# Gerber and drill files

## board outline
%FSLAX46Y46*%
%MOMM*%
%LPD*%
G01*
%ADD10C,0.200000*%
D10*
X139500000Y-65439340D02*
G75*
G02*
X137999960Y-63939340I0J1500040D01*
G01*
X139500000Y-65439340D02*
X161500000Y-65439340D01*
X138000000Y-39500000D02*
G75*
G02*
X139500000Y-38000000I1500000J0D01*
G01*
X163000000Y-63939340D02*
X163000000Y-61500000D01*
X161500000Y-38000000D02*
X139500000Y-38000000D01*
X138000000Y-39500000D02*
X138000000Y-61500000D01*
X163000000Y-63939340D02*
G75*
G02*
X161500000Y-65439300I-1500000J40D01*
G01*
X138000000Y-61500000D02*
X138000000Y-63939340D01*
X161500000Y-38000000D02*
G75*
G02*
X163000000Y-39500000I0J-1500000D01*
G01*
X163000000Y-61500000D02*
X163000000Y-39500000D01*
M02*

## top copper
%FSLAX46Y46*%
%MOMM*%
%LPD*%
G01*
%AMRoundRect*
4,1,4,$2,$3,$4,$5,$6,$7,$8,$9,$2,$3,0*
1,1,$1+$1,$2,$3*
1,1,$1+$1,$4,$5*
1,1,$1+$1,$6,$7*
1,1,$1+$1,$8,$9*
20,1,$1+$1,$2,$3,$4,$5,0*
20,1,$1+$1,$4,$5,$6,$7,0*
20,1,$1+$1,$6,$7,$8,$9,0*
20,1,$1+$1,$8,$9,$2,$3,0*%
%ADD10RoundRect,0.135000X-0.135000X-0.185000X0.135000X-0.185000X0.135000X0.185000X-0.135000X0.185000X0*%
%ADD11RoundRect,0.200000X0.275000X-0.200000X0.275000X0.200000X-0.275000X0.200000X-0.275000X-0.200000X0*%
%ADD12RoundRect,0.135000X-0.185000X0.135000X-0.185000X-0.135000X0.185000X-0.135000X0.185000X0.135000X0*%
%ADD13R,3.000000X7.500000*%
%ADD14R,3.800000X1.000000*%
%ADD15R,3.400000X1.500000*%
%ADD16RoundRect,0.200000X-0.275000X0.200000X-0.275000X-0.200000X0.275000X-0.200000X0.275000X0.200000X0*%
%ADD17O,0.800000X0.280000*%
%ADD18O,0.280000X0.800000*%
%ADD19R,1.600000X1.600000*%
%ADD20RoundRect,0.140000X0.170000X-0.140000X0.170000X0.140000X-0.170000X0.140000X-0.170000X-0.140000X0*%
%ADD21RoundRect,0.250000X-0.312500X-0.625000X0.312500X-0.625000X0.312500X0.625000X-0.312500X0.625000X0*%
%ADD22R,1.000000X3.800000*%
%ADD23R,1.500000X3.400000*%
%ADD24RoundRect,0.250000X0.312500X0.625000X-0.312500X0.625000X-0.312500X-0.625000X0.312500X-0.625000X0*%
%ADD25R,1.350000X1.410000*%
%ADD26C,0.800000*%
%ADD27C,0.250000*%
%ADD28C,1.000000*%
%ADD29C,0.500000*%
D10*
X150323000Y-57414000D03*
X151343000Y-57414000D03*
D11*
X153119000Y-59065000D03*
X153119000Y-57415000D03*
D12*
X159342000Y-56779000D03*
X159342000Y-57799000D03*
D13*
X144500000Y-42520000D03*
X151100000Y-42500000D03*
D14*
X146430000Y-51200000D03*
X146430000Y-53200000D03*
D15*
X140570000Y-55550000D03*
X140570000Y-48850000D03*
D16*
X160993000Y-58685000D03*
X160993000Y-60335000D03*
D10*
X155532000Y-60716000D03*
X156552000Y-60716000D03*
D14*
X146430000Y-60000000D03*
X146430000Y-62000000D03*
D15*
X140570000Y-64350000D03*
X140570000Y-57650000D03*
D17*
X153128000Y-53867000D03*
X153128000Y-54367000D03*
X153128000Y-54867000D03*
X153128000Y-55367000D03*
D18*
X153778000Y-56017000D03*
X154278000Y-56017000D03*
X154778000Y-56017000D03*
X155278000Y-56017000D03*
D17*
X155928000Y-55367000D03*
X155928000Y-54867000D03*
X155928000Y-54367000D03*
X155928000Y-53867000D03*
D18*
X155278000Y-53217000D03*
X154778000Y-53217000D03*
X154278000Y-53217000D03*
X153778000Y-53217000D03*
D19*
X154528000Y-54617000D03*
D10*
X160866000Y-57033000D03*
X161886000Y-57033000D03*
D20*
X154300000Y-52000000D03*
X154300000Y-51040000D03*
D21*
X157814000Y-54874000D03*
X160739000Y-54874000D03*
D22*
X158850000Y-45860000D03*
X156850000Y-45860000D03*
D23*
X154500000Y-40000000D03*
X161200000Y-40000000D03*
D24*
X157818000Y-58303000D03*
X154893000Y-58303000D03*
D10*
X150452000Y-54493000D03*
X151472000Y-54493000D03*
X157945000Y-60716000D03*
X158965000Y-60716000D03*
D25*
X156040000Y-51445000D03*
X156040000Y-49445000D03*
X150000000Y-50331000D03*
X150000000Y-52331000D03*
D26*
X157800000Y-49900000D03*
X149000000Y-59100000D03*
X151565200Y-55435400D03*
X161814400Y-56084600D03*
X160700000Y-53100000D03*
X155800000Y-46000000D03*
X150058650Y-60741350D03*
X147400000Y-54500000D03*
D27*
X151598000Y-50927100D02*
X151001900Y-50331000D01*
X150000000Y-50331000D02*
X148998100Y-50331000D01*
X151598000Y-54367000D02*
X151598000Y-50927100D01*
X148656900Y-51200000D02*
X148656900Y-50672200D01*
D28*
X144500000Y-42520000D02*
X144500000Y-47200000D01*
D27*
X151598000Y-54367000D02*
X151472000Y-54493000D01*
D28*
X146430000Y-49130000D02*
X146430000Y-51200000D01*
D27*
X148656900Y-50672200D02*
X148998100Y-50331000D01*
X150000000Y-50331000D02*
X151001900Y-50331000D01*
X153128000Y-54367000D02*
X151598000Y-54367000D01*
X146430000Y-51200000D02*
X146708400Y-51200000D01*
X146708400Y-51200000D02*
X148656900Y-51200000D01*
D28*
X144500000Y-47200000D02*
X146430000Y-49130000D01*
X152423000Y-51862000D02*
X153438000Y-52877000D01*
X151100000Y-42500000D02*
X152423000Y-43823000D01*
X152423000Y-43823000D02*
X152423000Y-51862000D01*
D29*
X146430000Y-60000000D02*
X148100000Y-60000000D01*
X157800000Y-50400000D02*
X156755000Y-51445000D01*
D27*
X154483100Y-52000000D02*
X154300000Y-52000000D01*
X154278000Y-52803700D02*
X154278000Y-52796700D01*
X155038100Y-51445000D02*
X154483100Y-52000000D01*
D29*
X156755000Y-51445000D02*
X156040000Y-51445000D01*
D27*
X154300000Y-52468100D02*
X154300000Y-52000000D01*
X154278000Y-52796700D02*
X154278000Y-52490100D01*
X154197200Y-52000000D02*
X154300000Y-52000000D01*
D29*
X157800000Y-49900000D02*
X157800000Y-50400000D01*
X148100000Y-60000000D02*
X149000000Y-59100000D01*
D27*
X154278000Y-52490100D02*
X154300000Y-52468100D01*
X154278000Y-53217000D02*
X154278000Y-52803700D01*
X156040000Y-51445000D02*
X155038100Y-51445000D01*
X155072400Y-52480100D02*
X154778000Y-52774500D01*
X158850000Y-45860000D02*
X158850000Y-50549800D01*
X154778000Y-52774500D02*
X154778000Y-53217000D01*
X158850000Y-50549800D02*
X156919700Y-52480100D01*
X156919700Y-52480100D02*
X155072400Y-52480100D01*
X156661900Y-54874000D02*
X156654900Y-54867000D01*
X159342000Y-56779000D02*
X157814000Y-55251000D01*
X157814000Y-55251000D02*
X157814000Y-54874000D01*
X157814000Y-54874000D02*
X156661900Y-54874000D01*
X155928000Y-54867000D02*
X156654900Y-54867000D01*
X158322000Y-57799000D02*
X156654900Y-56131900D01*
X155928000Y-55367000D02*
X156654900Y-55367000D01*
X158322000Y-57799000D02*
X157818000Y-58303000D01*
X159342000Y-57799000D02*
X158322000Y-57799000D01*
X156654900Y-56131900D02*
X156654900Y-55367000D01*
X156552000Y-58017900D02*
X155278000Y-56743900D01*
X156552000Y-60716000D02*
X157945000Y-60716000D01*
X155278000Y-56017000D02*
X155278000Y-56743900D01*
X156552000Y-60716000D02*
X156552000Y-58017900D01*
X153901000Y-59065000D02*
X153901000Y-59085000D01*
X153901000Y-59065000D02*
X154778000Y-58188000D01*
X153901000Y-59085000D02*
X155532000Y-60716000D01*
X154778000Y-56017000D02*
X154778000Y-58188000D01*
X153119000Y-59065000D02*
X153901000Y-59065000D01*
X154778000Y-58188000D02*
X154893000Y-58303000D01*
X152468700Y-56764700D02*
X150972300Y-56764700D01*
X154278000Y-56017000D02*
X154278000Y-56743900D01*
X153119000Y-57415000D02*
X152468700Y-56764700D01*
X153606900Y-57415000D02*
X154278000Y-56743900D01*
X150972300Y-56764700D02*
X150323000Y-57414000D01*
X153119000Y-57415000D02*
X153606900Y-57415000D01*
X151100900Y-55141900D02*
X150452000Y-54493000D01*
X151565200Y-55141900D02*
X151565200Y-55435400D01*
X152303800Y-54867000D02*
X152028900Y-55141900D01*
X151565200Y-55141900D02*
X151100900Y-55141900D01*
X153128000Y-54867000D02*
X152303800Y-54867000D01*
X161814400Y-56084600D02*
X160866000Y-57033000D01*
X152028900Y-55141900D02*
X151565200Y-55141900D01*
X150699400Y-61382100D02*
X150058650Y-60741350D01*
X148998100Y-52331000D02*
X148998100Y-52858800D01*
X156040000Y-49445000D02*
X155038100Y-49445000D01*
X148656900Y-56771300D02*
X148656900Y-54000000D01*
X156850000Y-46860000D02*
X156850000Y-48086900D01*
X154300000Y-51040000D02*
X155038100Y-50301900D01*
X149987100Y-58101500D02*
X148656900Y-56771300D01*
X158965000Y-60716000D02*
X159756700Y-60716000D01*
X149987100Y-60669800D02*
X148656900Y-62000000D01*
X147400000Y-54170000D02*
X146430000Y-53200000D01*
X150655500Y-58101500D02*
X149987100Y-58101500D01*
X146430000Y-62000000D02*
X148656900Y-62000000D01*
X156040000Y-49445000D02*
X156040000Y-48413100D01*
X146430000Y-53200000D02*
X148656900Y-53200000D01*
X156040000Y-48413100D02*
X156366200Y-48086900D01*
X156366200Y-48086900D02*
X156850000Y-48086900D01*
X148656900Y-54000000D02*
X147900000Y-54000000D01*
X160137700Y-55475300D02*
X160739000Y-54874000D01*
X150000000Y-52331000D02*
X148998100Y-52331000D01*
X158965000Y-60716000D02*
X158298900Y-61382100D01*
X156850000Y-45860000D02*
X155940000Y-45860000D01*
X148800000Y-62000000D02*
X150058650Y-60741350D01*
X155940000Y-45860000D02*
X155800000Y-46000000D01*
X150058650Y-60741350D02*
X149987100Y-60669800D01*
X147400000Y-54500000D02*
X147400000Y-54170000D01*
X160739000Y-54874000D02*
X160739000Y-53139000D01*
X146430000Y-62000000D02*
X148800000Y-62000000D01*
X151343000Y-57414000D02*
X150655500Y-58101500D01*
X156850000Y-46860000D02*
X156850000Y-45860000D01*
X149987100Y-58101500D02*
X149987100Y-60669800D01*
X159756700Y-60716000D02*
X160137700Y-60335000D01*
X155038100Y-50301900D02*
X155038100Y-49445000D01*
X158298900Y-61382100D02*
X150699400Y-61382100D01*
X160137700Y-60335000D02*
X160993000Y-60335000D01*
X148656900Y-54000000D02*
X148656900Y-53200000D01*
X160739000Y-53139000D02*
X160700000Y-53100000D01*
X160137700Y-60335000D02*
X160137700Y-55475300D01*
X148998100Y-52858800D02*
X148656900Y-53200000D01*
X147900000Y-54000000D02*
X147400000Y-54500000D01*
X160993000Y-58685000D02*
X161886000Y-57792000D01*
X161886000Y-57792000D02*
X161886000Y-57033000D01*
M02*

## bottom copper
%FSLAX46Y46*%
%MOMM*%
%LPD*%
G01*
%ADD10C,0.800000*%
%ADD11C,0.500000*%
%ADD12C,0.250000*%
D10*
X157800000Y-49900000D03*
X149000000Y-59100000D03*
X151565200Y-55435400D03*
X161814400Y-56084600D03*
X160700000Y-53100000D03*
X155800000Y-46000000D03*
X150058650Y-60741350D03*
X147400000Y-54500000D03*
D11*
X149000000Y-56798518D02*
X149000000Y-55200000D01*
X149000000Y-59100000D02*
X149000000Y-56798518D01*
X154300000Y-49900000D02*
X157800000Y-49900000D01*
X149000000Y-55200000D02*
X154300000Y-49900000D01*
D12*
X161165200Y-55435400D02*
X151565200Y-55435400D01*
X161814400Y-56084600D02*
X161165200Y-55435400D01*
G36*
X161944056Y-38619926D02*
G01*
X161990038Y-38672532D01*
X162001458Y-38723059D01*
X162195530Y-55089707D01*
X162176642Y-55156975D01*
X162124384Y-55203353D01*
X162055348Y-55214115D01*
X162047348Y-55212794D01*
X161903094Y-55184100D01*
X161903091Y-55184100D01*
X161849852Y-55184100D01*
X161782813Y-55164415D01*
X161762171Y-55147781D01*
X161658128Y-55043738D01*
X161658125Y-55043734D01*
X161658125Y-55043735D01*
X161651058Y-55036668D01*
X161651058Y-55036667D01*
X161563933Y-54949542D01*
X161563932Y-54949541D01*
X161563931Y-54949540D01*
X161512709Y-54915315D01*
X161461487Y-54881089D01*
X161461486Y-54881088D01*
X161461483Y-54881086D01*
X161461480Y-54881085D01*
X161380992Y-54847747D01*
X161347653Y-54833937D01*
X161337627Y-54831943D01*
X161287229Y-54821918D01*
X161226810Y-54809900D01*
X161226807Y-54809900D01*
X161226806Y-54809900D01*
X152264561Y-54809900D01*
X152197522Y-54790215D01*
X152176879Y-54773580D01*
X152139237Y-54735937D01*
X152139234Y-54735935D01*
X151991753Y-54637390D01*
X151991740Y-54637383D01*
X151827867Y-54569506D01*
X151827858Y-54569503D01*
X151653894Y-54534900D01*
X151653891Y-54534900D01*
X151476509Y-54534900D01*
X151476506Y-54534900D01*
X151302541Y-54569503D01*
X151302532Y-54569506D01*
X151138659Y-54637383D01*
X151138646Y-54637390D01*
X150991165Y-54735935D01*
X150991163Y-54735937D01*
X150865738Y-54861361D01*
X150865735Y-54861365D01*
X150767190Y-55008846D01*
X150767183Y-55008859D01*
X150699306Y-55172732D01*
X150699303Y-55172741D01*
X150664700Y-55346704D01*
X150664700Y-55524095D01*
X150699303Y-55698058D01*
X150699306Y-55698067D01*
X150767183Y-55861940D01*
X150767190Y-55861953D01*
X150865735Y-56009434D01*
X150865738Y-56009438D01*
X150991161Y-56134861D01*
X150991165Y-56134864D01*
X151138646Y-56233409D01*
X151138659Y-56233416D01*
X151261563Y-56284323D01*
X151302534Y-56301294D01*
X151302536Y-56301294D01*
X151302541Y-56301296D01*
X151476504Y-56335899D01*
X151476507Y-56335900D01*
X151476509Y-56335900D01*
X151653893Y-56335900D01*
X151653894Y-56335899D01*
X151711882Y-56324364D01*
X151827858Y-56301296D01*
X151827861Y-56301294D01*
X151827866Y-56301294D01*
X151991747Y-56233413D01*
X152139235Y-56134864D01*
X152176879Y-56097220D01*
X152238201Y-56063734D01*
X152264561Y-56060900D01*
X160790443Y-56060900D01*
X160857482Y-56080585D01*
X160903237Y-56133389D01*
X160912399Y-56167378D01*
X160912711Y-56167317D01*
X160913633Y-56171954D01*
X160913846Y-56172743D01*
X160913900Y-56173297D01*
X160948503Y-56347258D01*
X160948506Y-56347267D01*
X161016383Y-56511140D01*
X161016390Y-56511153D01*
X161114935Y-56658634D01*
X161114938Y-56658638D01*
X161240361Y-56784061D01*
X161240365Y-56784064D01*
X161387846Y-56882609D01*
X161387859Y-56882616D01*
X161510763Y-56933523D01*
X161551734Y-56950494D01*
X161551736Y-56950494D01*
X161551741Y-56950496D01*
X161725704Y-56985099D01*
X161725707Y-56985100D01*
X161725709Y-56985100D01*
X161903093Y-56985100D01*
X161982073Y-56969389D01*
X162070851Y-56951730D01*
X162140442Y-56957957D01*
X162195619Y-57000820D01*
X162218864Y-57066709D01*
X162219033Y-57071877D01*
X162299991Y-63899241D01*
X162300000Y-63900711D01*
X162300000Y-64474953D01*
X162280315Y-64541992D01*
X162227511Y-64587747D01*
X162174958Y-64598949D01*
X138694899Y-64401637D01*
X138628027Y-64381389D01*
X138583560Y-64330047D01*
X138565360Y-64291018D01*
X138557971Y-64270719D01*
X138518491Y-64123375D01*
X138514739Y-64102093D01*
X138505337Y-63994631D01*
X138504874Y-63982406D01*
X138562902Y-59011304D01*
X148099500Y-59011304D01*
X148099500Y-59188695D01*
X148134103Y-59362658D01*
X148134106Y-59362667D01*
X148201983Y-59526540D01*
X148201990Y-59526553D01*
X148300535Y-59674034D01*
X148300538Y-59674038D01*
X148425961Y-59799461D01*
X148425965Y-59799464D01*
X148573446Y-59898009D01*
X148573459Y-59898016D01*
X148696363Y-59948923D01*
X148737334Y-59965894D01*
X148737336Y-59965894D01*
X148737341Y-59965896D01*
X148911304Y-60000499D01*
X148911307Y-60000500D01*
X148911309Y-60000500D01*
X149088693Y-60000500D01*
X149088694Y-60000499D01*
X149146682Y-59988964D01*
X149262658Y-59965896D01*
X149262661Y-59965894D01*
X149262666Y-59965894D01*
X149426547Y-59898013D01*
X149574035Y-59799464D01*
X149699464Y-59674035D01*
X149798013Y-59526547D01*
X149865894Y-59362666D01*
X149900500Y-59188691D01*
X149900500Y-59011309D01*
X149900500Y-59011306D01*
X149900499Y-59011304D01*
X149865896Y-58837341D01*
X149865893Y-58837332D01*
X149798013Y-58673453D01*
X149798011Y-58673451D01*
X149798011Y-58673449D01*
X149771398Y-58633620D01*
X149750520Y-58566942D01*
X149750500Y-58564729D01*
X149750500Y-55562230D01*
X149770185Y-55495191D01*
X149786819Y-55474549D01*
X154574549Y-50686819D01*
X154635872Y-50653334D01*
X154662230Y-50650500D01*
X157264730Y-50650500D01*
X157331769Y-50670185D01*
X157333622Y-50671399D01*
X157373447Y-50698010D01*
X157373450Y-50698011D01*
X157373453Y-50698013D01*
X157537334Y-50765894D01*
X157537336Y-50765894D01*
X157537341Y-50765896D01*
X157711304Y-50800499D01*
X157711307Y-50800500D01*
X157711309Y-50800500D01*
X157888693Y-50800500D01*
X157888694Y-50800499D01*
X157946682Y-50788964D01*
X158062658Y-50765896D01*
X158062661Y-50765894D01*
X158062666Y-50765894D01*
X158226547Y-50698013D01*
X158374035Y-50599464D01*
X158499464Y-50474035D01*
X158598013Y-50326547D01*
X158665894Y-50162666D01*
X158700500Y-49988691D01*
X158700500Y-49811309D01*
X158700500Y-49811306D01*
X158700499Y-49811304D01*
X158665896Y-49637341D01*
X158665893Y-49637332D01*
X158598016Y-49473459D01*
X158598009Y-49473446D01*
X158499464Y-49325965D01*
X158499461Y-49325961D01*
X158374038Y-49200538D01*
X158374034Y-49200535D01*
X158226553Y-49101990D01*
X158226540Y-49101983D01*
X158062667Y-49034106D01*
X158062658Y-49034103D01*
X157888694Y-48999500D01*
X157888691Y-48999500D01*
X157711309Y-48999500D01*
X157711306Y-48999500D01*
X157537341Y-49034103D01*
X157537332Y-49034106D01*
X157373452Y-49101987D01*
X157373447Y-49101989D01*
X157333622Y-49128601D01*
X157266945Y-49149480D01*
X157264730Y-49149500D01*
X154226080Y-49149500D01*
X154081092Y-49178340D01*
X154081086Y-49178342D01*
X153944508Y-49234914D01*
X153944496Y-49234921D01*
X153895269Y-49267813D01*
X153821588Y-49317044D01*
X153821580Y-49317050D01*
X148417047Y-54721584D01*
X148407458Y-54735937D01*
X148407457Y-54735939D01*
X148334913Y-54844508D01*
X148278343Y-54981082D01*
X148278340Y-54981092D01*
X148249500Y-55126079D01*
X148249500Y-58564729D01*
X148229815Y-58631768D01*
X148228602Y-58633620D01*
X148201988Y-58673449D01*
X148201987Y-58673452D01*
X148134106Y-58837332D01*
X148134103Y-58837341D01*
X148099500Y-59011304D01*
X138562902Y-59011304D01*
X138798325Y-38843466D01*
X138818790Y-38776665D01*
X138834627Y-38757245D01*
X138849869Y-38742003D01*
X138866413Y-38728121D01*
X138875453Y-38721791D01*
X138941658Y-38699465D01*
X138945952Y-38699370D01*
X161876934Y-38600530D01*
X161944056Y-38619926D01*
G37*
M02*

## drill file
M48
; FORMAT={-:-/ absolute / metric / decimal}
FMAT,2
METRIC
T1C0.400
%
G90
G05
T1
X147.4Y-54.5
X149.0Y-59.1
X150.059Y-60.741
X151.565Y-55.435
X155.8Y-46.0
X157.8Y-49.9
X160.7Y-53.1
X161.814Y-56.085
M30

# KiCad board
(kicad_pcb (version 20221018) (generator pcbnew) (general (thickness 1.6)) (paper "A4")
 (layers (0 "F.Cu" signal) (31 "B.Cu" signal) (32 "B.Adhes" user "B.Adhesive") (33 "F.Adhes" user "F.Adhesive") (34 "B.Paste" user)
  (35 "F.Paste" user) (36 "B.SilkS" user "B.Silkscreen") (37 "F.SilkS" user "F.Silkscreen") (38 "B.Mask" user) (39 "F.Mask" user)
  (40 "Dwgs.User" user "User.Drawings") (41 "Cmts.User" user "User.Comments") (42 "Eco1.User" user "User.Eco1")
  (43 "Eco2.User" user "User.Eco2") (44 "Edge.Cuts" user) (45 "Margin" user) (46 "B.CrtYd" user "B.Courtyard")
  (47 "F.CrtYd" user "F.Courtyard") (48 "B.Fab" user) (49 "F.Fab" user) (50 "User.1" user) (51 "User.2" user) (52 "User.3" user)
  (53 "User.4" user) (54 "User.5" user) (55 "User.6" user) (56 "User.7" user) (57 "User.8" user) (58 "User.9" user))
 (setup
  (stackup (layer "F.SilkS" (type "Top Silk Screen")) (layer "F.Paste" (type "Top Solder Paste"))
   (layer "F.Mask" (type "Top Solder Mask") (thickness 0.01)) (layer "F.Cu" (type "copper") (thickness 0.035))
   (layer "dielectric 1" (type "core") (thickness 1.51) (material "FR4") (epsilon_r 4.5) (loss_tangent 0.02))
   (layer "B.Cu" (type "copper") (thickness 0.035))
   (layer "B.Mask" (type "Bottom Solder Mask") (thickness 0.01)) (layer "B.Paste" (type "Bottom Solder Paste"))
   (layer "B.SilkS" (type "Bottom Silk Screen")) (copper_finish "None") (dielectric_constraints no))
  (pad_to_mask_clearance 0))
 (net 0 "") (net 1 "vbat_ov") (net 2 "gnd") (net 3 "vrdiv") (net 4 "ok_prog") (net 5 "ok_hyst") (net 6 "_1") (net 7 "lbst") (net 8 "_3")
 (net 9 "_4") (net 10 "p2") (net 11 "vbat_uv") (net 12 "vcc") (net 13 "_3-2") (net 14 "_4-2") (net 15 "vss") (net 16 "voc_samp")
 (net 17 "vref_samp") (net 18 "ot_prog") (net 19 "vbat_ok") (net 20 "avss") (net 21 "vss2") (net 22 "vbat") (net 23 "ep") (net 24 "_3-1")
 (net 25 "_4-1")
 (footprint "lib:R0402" (layer "F.Cu") (at 150.833 57.414)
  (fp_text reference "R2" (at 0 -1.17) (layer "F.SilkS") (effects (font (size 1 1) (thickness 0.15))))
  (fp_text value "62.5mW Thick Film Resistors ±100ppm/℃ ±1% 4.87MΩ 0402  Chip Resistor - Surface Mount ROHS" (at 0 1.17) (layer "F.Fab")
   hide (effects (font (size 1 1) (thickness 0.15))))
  (pad "1" smd roundrect (at -0.51 0) (size 0.54 0.64) (layers "F.Cu" "F.Paste" "F.Mask") (roundrect_rratio 0.25) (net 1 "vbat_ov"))
  (pad "2" smd roundrect (at 0.51 0) (size 0.54 0.64) (layers "F.Cu" "F.Paste" "F.Mask") (roundrect_rratio 0.25) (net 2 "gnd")))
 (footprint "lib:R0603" (layer "F.Cu") (at 153.119 58.24 90)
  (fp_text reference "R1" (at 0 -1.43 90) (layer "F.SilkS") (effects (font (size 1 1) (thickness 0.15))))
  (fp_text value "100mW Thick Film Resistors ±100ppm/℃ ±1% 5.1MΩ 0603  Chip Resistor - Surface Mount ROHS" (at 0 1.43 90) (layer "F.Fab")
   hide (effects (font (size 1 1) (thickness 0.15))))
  (pad "1" smd roundrect (at -0.825 0 90) (size 0.8 0.95) (layers "F.Cu" "F.Paste" "F.Mask") (roundrect_rratio 0.25) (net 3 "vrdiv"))
  (pad "2" smd roundrect (at 0.825 0 90) (size 0.8 0.95) (layers "F.Cu" "F.Paste" "F.Mask") (roundrect_rratio 0.25) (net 1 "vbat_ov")))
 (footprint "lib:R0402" (layer "F.Cu") (at 159.342 57.289 -90)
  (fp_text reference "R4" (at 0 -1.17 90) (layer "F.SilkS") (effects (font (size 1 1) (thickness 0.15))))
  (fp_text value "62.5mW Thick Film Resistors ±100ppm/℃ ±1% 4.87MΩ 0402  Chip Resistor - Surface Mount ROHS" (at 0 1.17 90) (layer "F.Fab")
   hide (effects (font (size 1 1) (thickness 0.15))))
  (pad "1" smd roundrect (at -0.51 0 270) (size 0.54 0.64) (layers "F.Cu" "F.Paste" "F.Mask") (roundrect_rratio 0.25) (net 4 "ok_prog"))
  (pad "2" smd roundrect (at 0.51 0 270) (size 0.54 0.64) (layers "F.Cu" "F.Paste" "F.Mask") (roundrect_rratio 0.25) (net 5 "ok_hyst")))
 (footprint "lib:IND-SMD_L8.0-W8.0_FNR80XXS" (layer "F.Cu") (at 147.8 42.51)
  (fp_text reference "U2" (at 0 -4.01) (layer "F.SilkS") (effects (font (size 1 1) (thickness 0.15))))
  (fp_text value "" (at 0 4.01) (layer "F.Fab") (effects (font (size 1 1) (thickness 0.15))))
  (pad "1" smd rect (at -3.3 0.01) (size 3 7.5) (layers "F.Cu" "F.Paste" "F.Mask") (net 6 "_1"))
  (pad "2" smd rect (at 3.3 -0.01) (size 3 7.5) (layers "F.Cu" "F.Paste" "F.Mask") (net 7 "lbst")))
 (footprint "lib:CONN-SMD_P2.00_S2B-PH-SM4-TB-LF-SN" (layer "F.Cu") (at 143.5 52.2 -90)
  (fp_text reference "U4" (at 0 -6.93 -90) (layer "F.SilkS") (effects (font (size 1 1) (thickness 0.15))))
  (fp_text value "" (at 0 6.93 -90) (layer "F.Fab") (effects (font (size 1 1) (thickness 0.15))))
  (pad "1" smd rect (at -1 -2.93 270) (size 1 3.8) (layers "F.Cu" "F.Paste" "F.Mask") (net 6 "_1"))
  (pad "2" smd rect (at 1 -2.93 270) (size 1 3.8) (layers "F.Cu" "F.Paste" "F.Mask") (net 2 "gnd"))
  (pad "3" smd rect (at 3.35 2.93 270) (size 1.5 3.4) (layers "F.Cu" "F.Paste" "F.Mask") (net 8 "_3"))
  (pad "4" smd rect (at -3.35 2.93 270) (size 1.5 3.4) (layers "F.Cu" "F.Paste" "F.Mask") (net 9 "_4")))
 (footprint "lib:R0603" (layer "F.Cu") (at 160.993 59.51 -90)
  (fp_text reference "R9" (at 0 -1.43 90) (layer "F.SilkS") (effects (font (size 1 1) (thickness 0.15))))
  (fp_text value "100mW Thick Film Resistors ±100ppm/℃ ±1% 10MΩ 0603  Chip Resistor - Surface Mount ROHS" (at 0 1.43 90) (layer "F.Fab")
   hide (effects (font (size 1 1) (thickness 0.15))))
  (pad "1" smd roundrect (at -0.825 0 270) (size 0.8 0.95) (layers "F.Cu" "F.Paste" "F.Mask") (roundrect_rratio 0.25) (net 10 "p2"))
  (pad "2" smd roundrect (at 0.825 0 270) (size 0.8 0.95) (layers "F.Cu" "F.Paste" "F.Mask") (roundrect_rratio 0.25) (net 2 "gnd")))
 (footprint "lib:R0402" (layer "F.Cu") (at 156.042 60.716)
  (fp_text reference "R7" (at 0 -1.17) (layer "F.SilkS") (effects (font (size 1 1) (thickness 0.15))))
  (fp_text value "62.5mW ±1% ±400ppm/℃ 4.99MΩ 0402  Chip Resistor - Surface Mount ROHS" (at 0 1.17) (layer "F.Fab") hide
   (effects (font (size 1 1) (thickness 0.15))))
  (pad "1" smd roundrect (at -0.51 0) (size 0.54 0.64) (layers "F.Cu" "F.Paste" "F.Mask") (roundrect_rratio 0.25) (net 3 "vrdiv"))
  (pad "2" smd roundrect (at 0.51 0) (size 0.54 0.64) (layers "F.Cu" "F.Paste" "F.Mask") (roundrect_rratio 0.25) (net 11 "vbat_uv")))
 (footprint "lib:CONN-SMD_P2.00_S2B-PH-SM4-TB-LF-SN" (layer "F.Cu") (at 143.5 61 -90)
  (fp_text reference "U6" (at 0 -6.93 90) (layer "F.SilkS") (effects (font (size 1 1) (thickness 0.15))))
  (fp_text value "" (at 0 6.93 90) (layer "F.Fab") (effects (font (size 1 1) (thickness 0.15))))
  (pad "1" smd rect (at -1 -2.93 270) (size 1 3.8) (layers "F.Cu" "F.Paste" "F.Mask") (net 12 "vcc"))
  (pad "2" smd rect (at 1 -2.93 270) (size 1 3.8) (layers "F.Cu" "F.Paste" "F.Mask") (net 2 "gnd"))
  (pad "3" smd rect (at 3.35 2.93 270) (size 1.5 3.4) (layers "F.Cu" "F.Paste" "F.Mask") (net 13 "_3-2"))
  (pad "4" smd rect (at -3.35 2.93 270) (size 1.5 3.4) (layers "F.Cu" "F.Paste" "F.Mask") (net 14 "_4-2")))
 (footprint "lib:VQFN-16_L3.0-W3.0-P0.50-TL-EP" (layer "F.Cu") (at 154.528 54.617)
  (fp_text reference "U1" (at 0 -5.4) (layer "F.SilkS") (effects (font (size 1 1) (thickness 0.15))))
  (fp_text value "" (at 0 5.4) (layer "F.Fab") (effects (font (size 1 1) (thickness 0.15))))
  (pad "1" smd oval (at -1.4 -0.75 90) (size 0.28 0.8) (layers "F.Cu" "F.Paste" "F.Mask") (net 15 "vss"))
  (pad "2" smd oval (at -1.4 -0.25 90) (size 0.28 0.8) (layers "F.Cu" "F.Paste" "F.Mask") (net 6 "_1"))
  (pad "3" smd oval (at -1.4 0.25 90) (size 0.28 0.8) (layers "F.Cu" "F.Paste" "F.Mask") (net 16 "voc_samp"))
  (pad "4" smd oval (at -1.4 0.75 90) (size 0.28 0.8) (layers "F.Cu" "F.Paste" "F.Mask") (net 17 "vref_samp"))
  (pad "5" smd oval (at -0.75 1.4) (size 0.28 0.8) (layers "F.Cu" "F.Paste" "F.Mask") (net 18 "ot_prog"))
  (pad "6" smd oval (at -0.25 1.4) (size 0.28 0.8) (layers "F.Cu" "F.Paste" "F.Mask") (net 1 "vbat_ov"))
  (pad "7" smd oval (at 0.25 1.4) (size 0.28 0.8) (layers "F.Cu" "F.Paste" "F.Mask") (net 3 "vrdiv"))
  (pad "8" smd oval (at 0.75 1.4) (size 0.28 0.8) (layers "F.Cu" "F.Paste" "F.Mask") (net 11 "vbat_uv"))
  (pad "9" smd oval (at 1.4 0.75 90) (size 0.28 0.8) (layers "F.Cu" "F.Paste" "F.Mask") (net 5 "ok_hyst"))
  (pad "10" smd oval (at 1.4 0.25 90) (size 0.28 0.8) (layers "F.Cu" "F.Paste" "F.Mask") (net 4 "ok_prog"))
  (pad "11" smd oval (at 1.4 -0.25 90) (size 0.28 0.8) (layers "F.Cu" "F.Paste" "F.Mask") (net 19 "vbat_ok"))
  (pad "12" smd oval (at 1.4 -0.75 90) (size 0.28 0.8) (layers "F.Cu" "F.Paste" "F.Mask") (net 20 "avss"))
  (pad "13" smd oval (at 0.75 -1.4) (size 0.28 0.8) (layers "F.Cu" "F.Paste" "F.Mask") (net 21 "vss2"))
  (pad "14" smd oval (at 0.25 -1.4) (size 0.28 0.8) (layers "F.Cu" "F.Paste" "F.Mask") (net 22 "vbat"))
  (pad "15" smd oval (at -0.25 -1.4) (size 0.28 0.8) (layers "F.Cu" "F.Paste" "F.Mask") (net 12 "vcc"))
  (pad "16" smd oval (at -0.75 -1.4) (size 0.28 0.8) (layers "F.Cu" "F.Paste" "F.Mask") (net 7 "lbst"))
  (pad "17" smd rect (at 0 0) (size 1.6 1.6) (layers "F.Cu" "F.Paste" "F.Mask") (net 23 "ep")))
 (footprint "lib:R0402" (layer "F.Cu") (at 161.376 57.033)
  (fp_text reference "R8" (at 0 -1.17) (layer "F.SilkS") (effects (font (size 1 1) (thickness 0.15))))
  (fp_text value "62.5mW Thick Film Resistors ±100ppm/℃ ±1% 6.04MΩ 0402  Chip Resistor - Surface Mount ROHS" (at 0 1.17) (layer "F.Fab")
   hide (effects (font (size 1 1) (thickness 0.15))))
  (pad "1" smd roundrect (at -0.51 0) (size 0.54 0.64) (layers "F.Cu" "F.Paste" "F.Mask") (roundrect_rratio 0.25) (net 16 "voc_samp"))
  (pad "2" smd roundrect (at 0.51 0) (size 0.54 0.64) (layers "F.Cu" "F.Paste" "F.Mask") (roundrect_rratio 0.25) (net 10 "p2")))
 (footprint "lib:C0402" (layer "F.Cu") (at 154.3 51.52 90)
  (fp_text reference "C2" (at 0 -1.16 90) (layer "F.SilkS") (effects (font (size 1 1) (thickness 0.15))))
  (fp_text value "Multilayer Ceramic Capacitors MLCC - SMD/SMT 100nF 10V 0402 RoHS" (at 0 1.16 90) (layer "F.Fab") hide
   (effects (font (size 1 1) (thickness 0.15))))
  (pad "1" smd roundrect (at -0.48 0 90) (size 0.56 0.62) (layers "F.Cu" "F.Paste" "F.Mask") (roundrect_rratio 0.25) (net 12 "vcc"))
  (pad "2" smd roundrect (at 0.48 0 90) (size 0.56 0.62) (layers "F.Cu" "F.Paste" "F.Mask") (roundrect_rratio 0.25) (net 2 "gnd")))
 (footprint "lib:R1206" (layer "F.Cu") (at 159.2765 54.874)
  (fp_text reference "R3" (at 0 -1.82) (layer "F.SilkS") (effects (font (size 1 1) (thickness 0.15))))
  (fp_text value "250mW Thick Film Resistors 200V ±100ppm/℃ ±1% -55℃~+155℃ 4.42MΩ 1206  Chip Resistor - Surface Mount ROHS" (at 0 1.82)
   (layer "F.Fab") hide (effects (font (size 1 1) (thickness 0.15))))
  (pad "1" smd roundrect (at -1.4625 0) (size 1.125 1.75) (layers "F.Cu" "F.Paste" "F.Mask") (roundrect_rratio 0.2222222222)
   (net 4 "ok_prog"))
  (pad "2" smd roundrect (at 1.4625 0) (size 1.125 1.75) (layers "F.Cu" "F.Paste" "F.Mask") (roundrect_rratio 0.2222222222) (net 2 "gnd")))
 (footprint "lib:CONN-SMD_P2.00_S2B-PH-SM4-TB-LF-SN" (layer "F.Cu") (at 157.85 42.93 180)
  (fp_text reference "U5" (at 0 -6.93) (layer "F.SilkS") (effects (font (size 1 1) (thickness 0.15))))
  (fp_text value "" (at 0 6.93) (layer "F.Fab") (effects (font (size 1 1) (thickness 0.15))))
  (pad "1" smd rect (at -1 -2.93 180) (size 1 3.8) (layers "F.Cu" "F.Paste" "F.Mask") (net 22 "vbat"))
  (pad "2" smd rect (at 1 -2.93 180) (size 1 3.8) (layers "F.Cu" "F.Paste" "F.Mask") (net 2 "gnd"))
  (pad "3" smd rect (at 3.35 2.93 180) (size 1.5 3.4) (layers "F.Cu" "F.Paste" "F.Mask") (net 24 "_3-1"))
  (pad "4" smd rect (at -3.35 2.93 180) (size 1.5 3.4) (layers "F.Cu" "F.Paste" "F.Mask") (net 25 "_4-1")))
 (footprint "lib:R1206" (layer "F.Cu") (at 156.3555 58.303 180)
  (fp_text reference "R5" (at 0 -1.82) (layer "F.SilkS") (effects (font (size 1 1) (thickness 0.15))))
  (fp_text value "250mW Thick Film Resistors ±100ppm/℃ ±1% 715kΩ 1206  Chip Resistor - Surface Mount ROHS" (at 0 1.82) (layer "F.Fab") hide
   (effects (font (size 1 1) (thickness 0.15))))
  (pad "1" smd roundrect (at -1.4625 0 180) (size 1.125 1.75) (layers "F.Cu" "F.Paste" "F.Mask") (roundrect_rratio 0.2222222222)
   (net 5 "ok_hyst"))
  (pad "2" smd roundrect (at 1.4625 0 180) (size 1.125 1.75) (layers "F.Cu" "F.Paste" "F.Mask") (roundrect_rratio 0.2222222222)
   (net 3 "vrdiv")))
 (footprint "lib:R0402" (layer "F.Cu") (at 150.962 54.493)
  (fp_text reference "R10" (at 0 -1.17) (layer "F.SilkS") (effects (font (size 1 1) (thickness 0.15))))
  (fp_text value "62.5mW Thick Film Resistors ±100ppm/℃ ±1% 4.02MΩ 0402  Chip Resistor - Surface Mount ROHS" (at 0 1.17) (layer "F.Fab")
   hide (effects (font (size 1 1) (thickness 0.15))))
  (pad "1" smd roundrect (at -0.51 0) (size 0.54 0.64) (layers "F.Cu" "F.Paste" "F.Mask") (roundrect_rratio 0.25) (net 16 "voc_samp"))
  (pad "2" smd roundrect (at 0.51 0) (size 0.54 0.64) (layers "F.Cu" "F.Paste" "F.Mask") (roundrect_rratio 0.25) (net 6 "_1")))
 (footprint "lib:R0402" (layer "F.Cu") (at 158.455 60.716)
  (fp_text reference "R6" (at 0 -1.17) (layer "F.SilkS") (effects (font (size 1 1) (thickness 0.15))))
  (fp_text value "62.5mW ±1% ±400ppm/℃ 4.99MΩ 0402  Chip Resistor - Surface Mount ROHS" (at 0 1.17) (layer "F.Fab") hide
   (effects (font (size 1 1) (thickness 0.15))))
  (pad "1" smd roundrect (at -0.51 0) (size 0.54 0.64) (layers "F.Cu" "F.Paste" "F.Mask") (roundrect_rratio 0.25) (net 11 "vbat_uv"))
  (pad "2" smd roundrect (at 0.51 0) (size 0.54 0.64) (layers "F.Cu" "F.Paste" "F.Mask") (roundrect_rratio 0.25) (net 2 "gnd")))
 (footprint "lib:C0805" (layer "F.Cu") (at 156.04 50.445 90)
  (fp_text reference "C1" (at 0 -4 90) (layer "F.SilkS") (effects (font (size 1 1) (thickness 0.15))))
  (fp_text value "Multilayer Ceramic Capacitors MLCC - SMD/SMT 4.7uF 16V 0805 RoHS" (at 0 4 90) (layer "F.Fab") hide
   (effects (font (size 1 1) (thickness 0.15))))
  (pad "1" smd rect (at -1 0 90) (size 1.41 1.35) (layers "F.Cu" "F.Paste" "F.Mask") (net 12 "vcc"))
  (pad "2" smd rect (at 1 0 90) (size 1.41 1.35) (layers "F.Cu" "F.Paste" "F.Mask") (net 2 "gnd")))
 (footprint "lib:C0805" (layer "F.Cu") (at 150 51.331 -90)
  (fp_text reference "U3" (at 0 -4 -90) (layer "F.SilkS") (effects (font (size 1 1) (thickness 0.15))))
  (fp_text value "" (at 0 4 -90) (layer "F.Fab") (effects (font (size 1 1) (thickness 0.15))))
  (pad "1" smd rect (at -1 0 270) (size 1.41 1.35) (layers "F.Cu" "F.Paste" "F.Mask") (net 6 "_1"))
  (pad "2" smd rect (at 1 0 270) (size 1.41 1.35) (layers "F.Cu" "F.Paste" "F.Mask") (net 2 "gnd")))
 (gr_arc (start 139.5 65.43934) (mid 138.43934 65) (end 138 63.93934) (stroke (width 0.2) (type default)) (layer "Edge.Cuts"))
 (gr_line (start 139.5 65.43934) (end 161.5 65.43934) (stroke (width 0.2) (type default)) (layer "Edge.Cuts"))
 (gr_arc (start 138 39.5) (mid 138.43934 38.43934) (end 139.5 38) (stroke (width 0.2) (type default)) (layer "Edge.Cuts"))
 (gr_line (start 163 63.93934) (end 163 61.5) (stroke (width 0.2) (type default)) (layer "Edge.Cuts"))
 (gr_line (start 161.5 38) (end 139.5 38) (stroke (width 0.2) (type default)) (layer "Edge.Cuts"))
 (gr_line (start 138 39.5) (end 138 61.5) (stroke (width 0.2) (type default)) (layer "Edge.Cuts"))
 (gr_arc (start 163 63.93934) (mid 162.56066 65) (end 161.5 65.43934) (stroke (width 0.2) (type default)) (layer "Edge.Cuts"))
 (gr_line (start 138 61.5) (end 138 63.93934) (stroke (width 0.2) (type default)) (layer "Edge.Cuts"))
 (gr_arc (start 161.5 38) (mid 162.56066 38.43934) (end 163 39.5) (stroke (width 0.2) (type default)) (layer "Edge.Cuts"))
 (gr_line (start 163 61.5) (end 163 39.5) (stroke (width 0.2) (type default)) (layer "Edge.Cuts"))
 (segment (start 151.598 50.9271) (end 151.0019 50.331) (width 0.25) (layer "F.Cu") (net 6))
 (segment (start 150 50.331) (end 148.9981 50.331) (width 0.25) (layer "F.Cu") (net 6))
 (segment (start 151.598 54.367) (end 151.598 50.9271) (width 0.25) (layer "F.Cu") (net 6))
 (segment (start 148.6569 51.2) (end 148.6569 50.6722) (width 0.25) (layer "F.Cu") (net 6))
 (segment (start 144.5 42.52) (end 144.5 47.2) (width 1) (layer "F.Cu") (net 6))
 (segment (start 151.598 54.367) (end 151.472 54.493) (width 0.25) (layer "F.Cu") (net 6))
 (segment (start 146.43 49.13) (end 146.43 51.2) (width 1) (layer "F.Cu") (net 6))
 (segment (start 148.6569 50.6722) (end 148.9981 50.331) (width 0.25) (layer "F.Cu") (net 6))
 (segment (start 150 50.331) (end 151.0019 50.331) (width 0.25) (layer "F.Cu") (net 6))
 (segment (start 153.128 54.367) (end 151.598 54.367) (width 0.25) (layer "F.Cu") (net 6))
 (segment (start 146.43 51.2) (end 146.7084 51.2) (width 0.25) (layer "F.Cu") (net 6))
 (segment (start 146.7084 51.2) (end 148.6569 51.2) (width 0.25) (layer "F.Cu") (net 6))
 (segment (start 144.5 47.2) (end 146.43 49.13) (width 1) (layer "F.Cu") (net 6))
 (segment (start 152.423 51.862) (end 153.438 52.877) (width 1) (layer "F.Cu") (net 7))
 (segment (start 151.1 42.5) (end 152.423 43.823) (width 1) (layer "F.Cu") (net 7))
 (segment (start 152.423 43.823) (end 152.423 51.862) (width 1) (layer "F.Cu") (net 7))
 (segment (start 146.43 60) (end 148.1 60) (width 0.5) (layer "F.Cu") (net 12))
 (segment (start 157.8 50.4) (end 156.755 51.445) (width 0.5) (layer "F.Cu") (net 12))
 (segment (start 154.4831 52) (end 154.3 52) (width 0.25) (layer "F.Cu") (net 12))
 (segment (start 154.278 52.8037) (end 154.278 52.7967) (width 0.25) (layer "F.Cu") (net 12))
 (segment (start 155.0381 51.445) (end 154.4831 52) (width 0.25) (layer "F.Cu") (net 12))
 (segment (start 156.755 51.445) (end 156.04 51.445) (width 0.5) (layer "F.Cu") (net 12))
 (segment (start 154.3 52.4681) (end 154.3 52) (width 0.25) (layer "F.Cu") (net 12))
 (segment (start 154.278 52.7967) (end 154.278 52.4901) (width 0.25) (layer "F.Cu") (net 12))
 (segment (start 154.1972 52) (end 154.3 52) (width 0.25) (layer "F.Cu") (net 12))
 (segment (start 157.8 49.9) (end 157.8 50.4) (width 0.5) (layer "F.Cu") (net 12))
 (segment (start 148.1 60) (end 149 59.1) (width 0.5) (layer "F.Cu") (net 12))
 (segment (start 154.278 52.4901) (end 154.3 52.4681) (width 0.25) (layer "F.Cu") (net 12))
 (segment (start 154.278 53.217) (end 154.278 52.8037) (width 0.25) (layer "F.Cu") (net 12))
 (segment (start 156.04 51.445) (end 155.0381 51.445) (width 0.25) (layer "F.Cu") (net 12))
 (via (at 157.8 49.9) (size 0.8) (drill 0.4) (layers "F.Cu" "B.Cu") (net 12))
 (via (at 149 59.1) (size 0.8) (drill 0.4) (layers "F.Cu" "B.Cu") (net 12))
 (segment (start 149 56.798518) (end 149 55.2) (width 0.5) (layer "B.Cu") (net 12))
 (segment (start 149 59.1) (end 149 56.798518) (width 0.5) (layer "B.Cu") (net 12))
 (segment (start 154.3 49.9) (end 157.8 49.9) (width 0.5) (layer "B.Cu") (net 12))
 (segment (start 149 55.2) (end 154.3 49.9) (width 0.5) (layer "B.Cu") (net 12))
 (segment (start 155.0724 52.4801) (end 154.778 52.7745) (width 0.25) (layer "F.Cu") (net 22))
 (segment (start 158.85 45.86) (end 158.85 50.5498) (width 0.25) (layer "F.Cu") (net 22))
 (segment (start 154.778 52.7745) (end 154.778 53.217) (width 0.25) (layer "F.Cu") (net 22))
 (segment (start 158.85 50.5498) (end 156.9197 52.4801) (width 0.25) (layer "F.Cu") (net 22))
 (segment (start 156.9197 52.4801) (end 155.0724 52.4801) (width 0.25) (layer "F.Cu") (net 22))
 (segment (start 156.6619 54.874) (end 156.6549 54.867) (width 0.25) (layer "F.Cu") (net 4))
 (segment (start 159.342 56.779) (end 157.814 55.251) (width 0.25) (layer "F.Cu") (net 4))
 (segment (start 157.814 55.251) (end 157.814 54.874) (width 0.25) (layer "F.Cu") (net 4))
 (segment (start 157.814 54.874) (end 156.6619 54.874) (width 0.25) (layer "F.Cu") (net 4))
 (segment (start 155.928 54.867) (end 156.6549 54.867) (width 0.25) (layer "F.Cu") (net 4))
 (segment (start 158.322 57.799) (end 156.6549 56.1319) (width 0.25) (layer "F.Cu") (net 5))
 (segment (start 155.928 55.367) (end 156.6549 55.367) (width 0.25) (layer "F.Cu") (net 5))
 (segment (start 158.322 57.799) (end 157.818 58.303) (width 0.25) (layer "F.Cu") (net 5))
 (segment (start 159.342 57.799) (end 158.322 57.799) (width 0.25) (layer "F.Cu") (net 5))
 (segment (start 156.6549 56.1319) (end 156.6549 55.367) (width 0.25) (layer "F.Cu") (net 5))
 (segment (start 156.552 58.0179) (end 155.278 56.7439) (width 0.25) (layer "F.Cu") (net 11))
 (segment (start 156.552 60.716) (end 157.945 60.716) (width 0.25) (layer "F.Cu") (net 11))
 (segment (start 155.278 56.017) (end 155.278 56.7439) (width 0.25) (layer "F.Cu") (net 11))
 (segment (start 156.552 60.716) (end 156.552 58.0179) (width 0.25) (layer "F.Cu") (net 11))
 (segment (start 153.901 59.065) (end 153.901 59.085) (width 0.25) (layer "F.Cu") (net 3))
 (segment (start 153.901 59.065) (end 154.778 58.188) (width 0.25) (layer "F.Cu") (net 3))
 (segment (start 153.901 59.085) (end 155.532 60.716) (width 0.25) (layer "F.Cu") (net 3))
 (segment (start 154.778 56.017) (end 154.778 58.188) (width 0.25) (layer "F.Cu") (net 3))
 (segment (start 153.119 59.065) (end 153.901 59.065) (width 0.25) (layer "F.Cu") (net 3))
 (segment (start 154.778 58.188) (end 154.893 58.303) (width 0.25) (layer "F.Cu") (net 3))
 (segment (start 152.4687 56.7647) (end 150.9723 56.7647) (width 0.25) (layer "F.Cu") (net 1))
 (segment (start 154.278 56.017) (end 154.278 56.7439) (width 0.25) (layer "F.Cu") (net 1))
 (segment (start 153.119 57.415) (end 152.4687 56.7647) (width 0.25) (layer "F.Cu") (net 1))
 (segment (start 153.6069 57.415) (end 154.278 56.7439) (width 0.25) (layer "F.Cu") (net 1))
 (segment (start 150.9723 56.7647) (end 150.323 57.414) (width 0.25) (layer "F.Cu") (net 1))
 (segment (start 153.119 57.415) (end 153.6069 57.415) (width 0.25) (layer "F.Cu") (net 1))
 (segment (start 151.1009 55.1419) (end 150.452 54.493) (width 0.25) (layer "F.Cu") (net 16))
 (segment (start 151.5652 55.1419) (end 151.5652 55.4354) (width 0.25) (layer "F.Cu") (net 16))
 (segment (start 152.3038 54.867) (end 152.0289 55.1419) (width 0.25) (layer "F.Cu") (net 16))
 (segment (start 151.5652 55.1419) (end 151.1009 55.1419) (width 0.25) (layer "F.Cu") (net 16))
 (segment (start 153.128 54.867) (end 152.3038 54.867) (width 0.25) (layer "F.Cu") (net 16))
 (segment (start 161.8144 56.0846) (end 160.866 57.033) (width 0.25) (layer "F.Cu") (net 16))
 (segment (start 152.0289 55.1419) (end 151.5652 55.1419) (width 0.25) (layer "F.Cu") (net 16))
 (via (at 151.5652 55.4354) (size 0.8) (drill 0.4) (layers "F.Cu" "B.Cu") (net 16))
 (via (at 161.8144 56.0846) (size 0.8) (drill 0.4) (layers "F.Cu" "B.Cu") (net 16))
 (segment (start 161.1652 55.4354) (end 151.5652 55.4354) (width 0.25) (layer "B.Cu") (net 16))
 (segment (start 161.8144 56.0846) (end 161.1652 55.4354) (width 0.25) (layer "B.Cu") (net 16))
 (segment (start 150.6994 61.3821) (end 150.05865 60.74135) (width 0.25) (layer "F.Cu") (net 2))
 (segment (start 148.9981 52.331) (end 148.9981 52.8588) (width 0.25) (layer "F.Cu") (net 2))
 (segment (start 156.04 49.445) (end 155.0381 49.445) (width 0.25) (layer "F.Cu") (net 2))
 (segment (start 148.6569 56.7713) (end 148.6569 54) (width 0.25) (layer "F.Cu") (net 2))
 (segment (start 156.85 46.86) (end 156.85 48.0869) (width 0.25) (layer "F.Cu") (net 2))
 (segment (start 154.3 51.04) (end 155.0381 50.3019) (width 0.25) (layer "F.Cu") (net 2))
 (segment (start 149.9871 58.1015) (end 148.6569 56.7713) (width 0.25) (layer "F.Cu") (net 2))
 (segment (start 158.965 60.716) (end 159.7567 60.716) (width 0.25) (layer "F.Cu") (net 2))
 (segment (start 149.9871 60.6698) (end 148.6569 62) (width 0.25) (layer "F.Cu") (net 2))
 (segment (start 147.4 54.17) (end 146.43 53.2) (width 0.25) (layer "F.Cu") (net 2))
 (segment (start 150.6555 58.1015) (end 149.9871 58.1015) (width 0.25) (layer "F.Cu") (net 2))
 (segment (start 146.43 62) (end 148.6569 62) (width 0.25) (layer "F.Cu") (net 2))
 (segment (start 156.04 49.445) (end 156.04 48.4131) (width 0.25) (layer "F.Cu") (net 2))
 (segment (start 146.43 53.2) (end 148.6569 53.2) (width 0.25) (layer "F.Cu") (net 2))
 (segment (start 156.04 48.4131) (end 156.3662 48.0869) (width 0.25) (layer "F.Cu") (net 2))
 (segment (start 156.3662 48.0869) (end 156.85 48.0869) (width 0.25) (layer "F.Cu") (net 2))
 (segment (start 148.6569 54) (end 147.9 54) (width 0.25) (layer "F.Cu") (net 2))
 (segment (start 160.1377 55.4753) (end 160.739 54.874) (width 0.25) (layer "F.Cu") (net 2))
 (segment (start 150 52.331) (end 148.9981 52.331) (width 0.25) (layer "F.Cu") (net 2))
 (segment (start 158.965 60.716) (end 158.2989 61.3821) (width 0.25) (layer "F.Cu") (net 2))
 (segment (start 156.85 45.86) (end 155.94 45.86) (width 0.25) (layer "F.Cu") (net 2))
 (segment (start 148.8 62) (end 150.05865 60.74135) (width 0.25) (layer "F.Cu") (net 2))
 (segment (start 155.94 45.86) (end 155.8 46) (width 0.25) (layer "F.Cu") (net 2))
 (segment (start 150.05865 60.74135) (end 149.9871 60.6698) (width 0.25) (layer "F.Cu") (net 2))
 (segment (start 147.4 54.5) (end 147.4 54.17) (width 0.25) (layer "F.Cu") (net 2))
 (segment (start 160.739 54.874) (end 160.739 53.139) (width 0.25) (layer "F.Cu") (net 2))
 (segment (start 146.43 62) (end 148.8 62) (width 0.25) (layer "F.Cu") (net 2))
 (segment (start 151.343 57.414) (end 150.6555 58.1015) (width 0.25) (layer "F.Cu") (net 2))
 (segment (start 156.85 46.86) (end 156.85 45.86) (width 0.25) (layer "F.Cu") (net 2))
 (segment (start 149.9871 58.1015) (end 149.9871 60.6698) (width 0.25) (layer "F.Cu") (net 2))
 (segment (start 159.7567 60.716) (end 160.1377 60.335) (width 0.25) (layer "F.Cu") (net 2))
 (segment (start 155.0381 50.3019) (end 155.0381 49.445) (width 0.25) (layer "F.Cu") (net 2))
 (segment (start 158.2989 61.3821) (end 150.6994 61.3821) (width 0.25) (layer "F.Cu") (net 2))
 (segment (start 160.1377 60.335) (end 160.993 60.335) (width 0.25) (layer "F.Cu") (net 2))
 (segment (start 148.6569 54) (end 148.6569 53.2) (width 0.25) (layer "F.Cu") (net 2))
 (segment (start 160.739 53.139) (end 160.7 53.1) (width 0.25) (layer "F.Cu") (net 2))
 (segment (start 160.1377 60.335) (end 160.1377 55.4753) (width 0.25) (layer "F.Cu") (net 2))
 (segment (start 148.9981 52.8588) (end 148.6569 53.2) (width 0.25) (layer "F.Cu") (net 2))
 (segment (start 147.9 54) (end 147.4 54.5) (width 0.25) (layer "F.Cu") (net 2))
 (via (at 160.7 53.1) (size 0.8) (drill 0.4) (layers "F.Cu" "B.Cu") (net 2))
 (via (at 155.8 46) (size 0.8) (drill 0.4) (layers "F.Cu" "B.Cu") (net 2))
 (via (at 150.05865 60.74135) (size 0.8) (drill 0.4) (layers "F.Cu" "B.Cu") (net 2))
 (via (at 147.4 54.5) (size 0.8) (drill 0.4) (layers "F.Cu" "B.Cu") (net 2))
 (segment (start 160.993 58.685) (end 161.886 57.792) (width 0.25) (layer "F.Cu") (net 10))
 (segment (start 161.886 57.792) (end 161.886 57.033) (width 0.25) (layer "F.Cu") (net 10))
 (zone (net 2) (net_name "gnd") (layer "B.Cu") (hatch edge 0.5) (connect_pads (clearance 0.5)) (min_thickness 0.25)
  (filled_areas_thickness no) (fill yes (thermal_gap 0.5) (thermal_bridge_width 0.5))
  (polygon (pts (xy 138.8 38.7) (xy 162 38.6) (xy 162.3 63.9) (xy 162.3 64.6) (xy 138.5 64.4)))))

